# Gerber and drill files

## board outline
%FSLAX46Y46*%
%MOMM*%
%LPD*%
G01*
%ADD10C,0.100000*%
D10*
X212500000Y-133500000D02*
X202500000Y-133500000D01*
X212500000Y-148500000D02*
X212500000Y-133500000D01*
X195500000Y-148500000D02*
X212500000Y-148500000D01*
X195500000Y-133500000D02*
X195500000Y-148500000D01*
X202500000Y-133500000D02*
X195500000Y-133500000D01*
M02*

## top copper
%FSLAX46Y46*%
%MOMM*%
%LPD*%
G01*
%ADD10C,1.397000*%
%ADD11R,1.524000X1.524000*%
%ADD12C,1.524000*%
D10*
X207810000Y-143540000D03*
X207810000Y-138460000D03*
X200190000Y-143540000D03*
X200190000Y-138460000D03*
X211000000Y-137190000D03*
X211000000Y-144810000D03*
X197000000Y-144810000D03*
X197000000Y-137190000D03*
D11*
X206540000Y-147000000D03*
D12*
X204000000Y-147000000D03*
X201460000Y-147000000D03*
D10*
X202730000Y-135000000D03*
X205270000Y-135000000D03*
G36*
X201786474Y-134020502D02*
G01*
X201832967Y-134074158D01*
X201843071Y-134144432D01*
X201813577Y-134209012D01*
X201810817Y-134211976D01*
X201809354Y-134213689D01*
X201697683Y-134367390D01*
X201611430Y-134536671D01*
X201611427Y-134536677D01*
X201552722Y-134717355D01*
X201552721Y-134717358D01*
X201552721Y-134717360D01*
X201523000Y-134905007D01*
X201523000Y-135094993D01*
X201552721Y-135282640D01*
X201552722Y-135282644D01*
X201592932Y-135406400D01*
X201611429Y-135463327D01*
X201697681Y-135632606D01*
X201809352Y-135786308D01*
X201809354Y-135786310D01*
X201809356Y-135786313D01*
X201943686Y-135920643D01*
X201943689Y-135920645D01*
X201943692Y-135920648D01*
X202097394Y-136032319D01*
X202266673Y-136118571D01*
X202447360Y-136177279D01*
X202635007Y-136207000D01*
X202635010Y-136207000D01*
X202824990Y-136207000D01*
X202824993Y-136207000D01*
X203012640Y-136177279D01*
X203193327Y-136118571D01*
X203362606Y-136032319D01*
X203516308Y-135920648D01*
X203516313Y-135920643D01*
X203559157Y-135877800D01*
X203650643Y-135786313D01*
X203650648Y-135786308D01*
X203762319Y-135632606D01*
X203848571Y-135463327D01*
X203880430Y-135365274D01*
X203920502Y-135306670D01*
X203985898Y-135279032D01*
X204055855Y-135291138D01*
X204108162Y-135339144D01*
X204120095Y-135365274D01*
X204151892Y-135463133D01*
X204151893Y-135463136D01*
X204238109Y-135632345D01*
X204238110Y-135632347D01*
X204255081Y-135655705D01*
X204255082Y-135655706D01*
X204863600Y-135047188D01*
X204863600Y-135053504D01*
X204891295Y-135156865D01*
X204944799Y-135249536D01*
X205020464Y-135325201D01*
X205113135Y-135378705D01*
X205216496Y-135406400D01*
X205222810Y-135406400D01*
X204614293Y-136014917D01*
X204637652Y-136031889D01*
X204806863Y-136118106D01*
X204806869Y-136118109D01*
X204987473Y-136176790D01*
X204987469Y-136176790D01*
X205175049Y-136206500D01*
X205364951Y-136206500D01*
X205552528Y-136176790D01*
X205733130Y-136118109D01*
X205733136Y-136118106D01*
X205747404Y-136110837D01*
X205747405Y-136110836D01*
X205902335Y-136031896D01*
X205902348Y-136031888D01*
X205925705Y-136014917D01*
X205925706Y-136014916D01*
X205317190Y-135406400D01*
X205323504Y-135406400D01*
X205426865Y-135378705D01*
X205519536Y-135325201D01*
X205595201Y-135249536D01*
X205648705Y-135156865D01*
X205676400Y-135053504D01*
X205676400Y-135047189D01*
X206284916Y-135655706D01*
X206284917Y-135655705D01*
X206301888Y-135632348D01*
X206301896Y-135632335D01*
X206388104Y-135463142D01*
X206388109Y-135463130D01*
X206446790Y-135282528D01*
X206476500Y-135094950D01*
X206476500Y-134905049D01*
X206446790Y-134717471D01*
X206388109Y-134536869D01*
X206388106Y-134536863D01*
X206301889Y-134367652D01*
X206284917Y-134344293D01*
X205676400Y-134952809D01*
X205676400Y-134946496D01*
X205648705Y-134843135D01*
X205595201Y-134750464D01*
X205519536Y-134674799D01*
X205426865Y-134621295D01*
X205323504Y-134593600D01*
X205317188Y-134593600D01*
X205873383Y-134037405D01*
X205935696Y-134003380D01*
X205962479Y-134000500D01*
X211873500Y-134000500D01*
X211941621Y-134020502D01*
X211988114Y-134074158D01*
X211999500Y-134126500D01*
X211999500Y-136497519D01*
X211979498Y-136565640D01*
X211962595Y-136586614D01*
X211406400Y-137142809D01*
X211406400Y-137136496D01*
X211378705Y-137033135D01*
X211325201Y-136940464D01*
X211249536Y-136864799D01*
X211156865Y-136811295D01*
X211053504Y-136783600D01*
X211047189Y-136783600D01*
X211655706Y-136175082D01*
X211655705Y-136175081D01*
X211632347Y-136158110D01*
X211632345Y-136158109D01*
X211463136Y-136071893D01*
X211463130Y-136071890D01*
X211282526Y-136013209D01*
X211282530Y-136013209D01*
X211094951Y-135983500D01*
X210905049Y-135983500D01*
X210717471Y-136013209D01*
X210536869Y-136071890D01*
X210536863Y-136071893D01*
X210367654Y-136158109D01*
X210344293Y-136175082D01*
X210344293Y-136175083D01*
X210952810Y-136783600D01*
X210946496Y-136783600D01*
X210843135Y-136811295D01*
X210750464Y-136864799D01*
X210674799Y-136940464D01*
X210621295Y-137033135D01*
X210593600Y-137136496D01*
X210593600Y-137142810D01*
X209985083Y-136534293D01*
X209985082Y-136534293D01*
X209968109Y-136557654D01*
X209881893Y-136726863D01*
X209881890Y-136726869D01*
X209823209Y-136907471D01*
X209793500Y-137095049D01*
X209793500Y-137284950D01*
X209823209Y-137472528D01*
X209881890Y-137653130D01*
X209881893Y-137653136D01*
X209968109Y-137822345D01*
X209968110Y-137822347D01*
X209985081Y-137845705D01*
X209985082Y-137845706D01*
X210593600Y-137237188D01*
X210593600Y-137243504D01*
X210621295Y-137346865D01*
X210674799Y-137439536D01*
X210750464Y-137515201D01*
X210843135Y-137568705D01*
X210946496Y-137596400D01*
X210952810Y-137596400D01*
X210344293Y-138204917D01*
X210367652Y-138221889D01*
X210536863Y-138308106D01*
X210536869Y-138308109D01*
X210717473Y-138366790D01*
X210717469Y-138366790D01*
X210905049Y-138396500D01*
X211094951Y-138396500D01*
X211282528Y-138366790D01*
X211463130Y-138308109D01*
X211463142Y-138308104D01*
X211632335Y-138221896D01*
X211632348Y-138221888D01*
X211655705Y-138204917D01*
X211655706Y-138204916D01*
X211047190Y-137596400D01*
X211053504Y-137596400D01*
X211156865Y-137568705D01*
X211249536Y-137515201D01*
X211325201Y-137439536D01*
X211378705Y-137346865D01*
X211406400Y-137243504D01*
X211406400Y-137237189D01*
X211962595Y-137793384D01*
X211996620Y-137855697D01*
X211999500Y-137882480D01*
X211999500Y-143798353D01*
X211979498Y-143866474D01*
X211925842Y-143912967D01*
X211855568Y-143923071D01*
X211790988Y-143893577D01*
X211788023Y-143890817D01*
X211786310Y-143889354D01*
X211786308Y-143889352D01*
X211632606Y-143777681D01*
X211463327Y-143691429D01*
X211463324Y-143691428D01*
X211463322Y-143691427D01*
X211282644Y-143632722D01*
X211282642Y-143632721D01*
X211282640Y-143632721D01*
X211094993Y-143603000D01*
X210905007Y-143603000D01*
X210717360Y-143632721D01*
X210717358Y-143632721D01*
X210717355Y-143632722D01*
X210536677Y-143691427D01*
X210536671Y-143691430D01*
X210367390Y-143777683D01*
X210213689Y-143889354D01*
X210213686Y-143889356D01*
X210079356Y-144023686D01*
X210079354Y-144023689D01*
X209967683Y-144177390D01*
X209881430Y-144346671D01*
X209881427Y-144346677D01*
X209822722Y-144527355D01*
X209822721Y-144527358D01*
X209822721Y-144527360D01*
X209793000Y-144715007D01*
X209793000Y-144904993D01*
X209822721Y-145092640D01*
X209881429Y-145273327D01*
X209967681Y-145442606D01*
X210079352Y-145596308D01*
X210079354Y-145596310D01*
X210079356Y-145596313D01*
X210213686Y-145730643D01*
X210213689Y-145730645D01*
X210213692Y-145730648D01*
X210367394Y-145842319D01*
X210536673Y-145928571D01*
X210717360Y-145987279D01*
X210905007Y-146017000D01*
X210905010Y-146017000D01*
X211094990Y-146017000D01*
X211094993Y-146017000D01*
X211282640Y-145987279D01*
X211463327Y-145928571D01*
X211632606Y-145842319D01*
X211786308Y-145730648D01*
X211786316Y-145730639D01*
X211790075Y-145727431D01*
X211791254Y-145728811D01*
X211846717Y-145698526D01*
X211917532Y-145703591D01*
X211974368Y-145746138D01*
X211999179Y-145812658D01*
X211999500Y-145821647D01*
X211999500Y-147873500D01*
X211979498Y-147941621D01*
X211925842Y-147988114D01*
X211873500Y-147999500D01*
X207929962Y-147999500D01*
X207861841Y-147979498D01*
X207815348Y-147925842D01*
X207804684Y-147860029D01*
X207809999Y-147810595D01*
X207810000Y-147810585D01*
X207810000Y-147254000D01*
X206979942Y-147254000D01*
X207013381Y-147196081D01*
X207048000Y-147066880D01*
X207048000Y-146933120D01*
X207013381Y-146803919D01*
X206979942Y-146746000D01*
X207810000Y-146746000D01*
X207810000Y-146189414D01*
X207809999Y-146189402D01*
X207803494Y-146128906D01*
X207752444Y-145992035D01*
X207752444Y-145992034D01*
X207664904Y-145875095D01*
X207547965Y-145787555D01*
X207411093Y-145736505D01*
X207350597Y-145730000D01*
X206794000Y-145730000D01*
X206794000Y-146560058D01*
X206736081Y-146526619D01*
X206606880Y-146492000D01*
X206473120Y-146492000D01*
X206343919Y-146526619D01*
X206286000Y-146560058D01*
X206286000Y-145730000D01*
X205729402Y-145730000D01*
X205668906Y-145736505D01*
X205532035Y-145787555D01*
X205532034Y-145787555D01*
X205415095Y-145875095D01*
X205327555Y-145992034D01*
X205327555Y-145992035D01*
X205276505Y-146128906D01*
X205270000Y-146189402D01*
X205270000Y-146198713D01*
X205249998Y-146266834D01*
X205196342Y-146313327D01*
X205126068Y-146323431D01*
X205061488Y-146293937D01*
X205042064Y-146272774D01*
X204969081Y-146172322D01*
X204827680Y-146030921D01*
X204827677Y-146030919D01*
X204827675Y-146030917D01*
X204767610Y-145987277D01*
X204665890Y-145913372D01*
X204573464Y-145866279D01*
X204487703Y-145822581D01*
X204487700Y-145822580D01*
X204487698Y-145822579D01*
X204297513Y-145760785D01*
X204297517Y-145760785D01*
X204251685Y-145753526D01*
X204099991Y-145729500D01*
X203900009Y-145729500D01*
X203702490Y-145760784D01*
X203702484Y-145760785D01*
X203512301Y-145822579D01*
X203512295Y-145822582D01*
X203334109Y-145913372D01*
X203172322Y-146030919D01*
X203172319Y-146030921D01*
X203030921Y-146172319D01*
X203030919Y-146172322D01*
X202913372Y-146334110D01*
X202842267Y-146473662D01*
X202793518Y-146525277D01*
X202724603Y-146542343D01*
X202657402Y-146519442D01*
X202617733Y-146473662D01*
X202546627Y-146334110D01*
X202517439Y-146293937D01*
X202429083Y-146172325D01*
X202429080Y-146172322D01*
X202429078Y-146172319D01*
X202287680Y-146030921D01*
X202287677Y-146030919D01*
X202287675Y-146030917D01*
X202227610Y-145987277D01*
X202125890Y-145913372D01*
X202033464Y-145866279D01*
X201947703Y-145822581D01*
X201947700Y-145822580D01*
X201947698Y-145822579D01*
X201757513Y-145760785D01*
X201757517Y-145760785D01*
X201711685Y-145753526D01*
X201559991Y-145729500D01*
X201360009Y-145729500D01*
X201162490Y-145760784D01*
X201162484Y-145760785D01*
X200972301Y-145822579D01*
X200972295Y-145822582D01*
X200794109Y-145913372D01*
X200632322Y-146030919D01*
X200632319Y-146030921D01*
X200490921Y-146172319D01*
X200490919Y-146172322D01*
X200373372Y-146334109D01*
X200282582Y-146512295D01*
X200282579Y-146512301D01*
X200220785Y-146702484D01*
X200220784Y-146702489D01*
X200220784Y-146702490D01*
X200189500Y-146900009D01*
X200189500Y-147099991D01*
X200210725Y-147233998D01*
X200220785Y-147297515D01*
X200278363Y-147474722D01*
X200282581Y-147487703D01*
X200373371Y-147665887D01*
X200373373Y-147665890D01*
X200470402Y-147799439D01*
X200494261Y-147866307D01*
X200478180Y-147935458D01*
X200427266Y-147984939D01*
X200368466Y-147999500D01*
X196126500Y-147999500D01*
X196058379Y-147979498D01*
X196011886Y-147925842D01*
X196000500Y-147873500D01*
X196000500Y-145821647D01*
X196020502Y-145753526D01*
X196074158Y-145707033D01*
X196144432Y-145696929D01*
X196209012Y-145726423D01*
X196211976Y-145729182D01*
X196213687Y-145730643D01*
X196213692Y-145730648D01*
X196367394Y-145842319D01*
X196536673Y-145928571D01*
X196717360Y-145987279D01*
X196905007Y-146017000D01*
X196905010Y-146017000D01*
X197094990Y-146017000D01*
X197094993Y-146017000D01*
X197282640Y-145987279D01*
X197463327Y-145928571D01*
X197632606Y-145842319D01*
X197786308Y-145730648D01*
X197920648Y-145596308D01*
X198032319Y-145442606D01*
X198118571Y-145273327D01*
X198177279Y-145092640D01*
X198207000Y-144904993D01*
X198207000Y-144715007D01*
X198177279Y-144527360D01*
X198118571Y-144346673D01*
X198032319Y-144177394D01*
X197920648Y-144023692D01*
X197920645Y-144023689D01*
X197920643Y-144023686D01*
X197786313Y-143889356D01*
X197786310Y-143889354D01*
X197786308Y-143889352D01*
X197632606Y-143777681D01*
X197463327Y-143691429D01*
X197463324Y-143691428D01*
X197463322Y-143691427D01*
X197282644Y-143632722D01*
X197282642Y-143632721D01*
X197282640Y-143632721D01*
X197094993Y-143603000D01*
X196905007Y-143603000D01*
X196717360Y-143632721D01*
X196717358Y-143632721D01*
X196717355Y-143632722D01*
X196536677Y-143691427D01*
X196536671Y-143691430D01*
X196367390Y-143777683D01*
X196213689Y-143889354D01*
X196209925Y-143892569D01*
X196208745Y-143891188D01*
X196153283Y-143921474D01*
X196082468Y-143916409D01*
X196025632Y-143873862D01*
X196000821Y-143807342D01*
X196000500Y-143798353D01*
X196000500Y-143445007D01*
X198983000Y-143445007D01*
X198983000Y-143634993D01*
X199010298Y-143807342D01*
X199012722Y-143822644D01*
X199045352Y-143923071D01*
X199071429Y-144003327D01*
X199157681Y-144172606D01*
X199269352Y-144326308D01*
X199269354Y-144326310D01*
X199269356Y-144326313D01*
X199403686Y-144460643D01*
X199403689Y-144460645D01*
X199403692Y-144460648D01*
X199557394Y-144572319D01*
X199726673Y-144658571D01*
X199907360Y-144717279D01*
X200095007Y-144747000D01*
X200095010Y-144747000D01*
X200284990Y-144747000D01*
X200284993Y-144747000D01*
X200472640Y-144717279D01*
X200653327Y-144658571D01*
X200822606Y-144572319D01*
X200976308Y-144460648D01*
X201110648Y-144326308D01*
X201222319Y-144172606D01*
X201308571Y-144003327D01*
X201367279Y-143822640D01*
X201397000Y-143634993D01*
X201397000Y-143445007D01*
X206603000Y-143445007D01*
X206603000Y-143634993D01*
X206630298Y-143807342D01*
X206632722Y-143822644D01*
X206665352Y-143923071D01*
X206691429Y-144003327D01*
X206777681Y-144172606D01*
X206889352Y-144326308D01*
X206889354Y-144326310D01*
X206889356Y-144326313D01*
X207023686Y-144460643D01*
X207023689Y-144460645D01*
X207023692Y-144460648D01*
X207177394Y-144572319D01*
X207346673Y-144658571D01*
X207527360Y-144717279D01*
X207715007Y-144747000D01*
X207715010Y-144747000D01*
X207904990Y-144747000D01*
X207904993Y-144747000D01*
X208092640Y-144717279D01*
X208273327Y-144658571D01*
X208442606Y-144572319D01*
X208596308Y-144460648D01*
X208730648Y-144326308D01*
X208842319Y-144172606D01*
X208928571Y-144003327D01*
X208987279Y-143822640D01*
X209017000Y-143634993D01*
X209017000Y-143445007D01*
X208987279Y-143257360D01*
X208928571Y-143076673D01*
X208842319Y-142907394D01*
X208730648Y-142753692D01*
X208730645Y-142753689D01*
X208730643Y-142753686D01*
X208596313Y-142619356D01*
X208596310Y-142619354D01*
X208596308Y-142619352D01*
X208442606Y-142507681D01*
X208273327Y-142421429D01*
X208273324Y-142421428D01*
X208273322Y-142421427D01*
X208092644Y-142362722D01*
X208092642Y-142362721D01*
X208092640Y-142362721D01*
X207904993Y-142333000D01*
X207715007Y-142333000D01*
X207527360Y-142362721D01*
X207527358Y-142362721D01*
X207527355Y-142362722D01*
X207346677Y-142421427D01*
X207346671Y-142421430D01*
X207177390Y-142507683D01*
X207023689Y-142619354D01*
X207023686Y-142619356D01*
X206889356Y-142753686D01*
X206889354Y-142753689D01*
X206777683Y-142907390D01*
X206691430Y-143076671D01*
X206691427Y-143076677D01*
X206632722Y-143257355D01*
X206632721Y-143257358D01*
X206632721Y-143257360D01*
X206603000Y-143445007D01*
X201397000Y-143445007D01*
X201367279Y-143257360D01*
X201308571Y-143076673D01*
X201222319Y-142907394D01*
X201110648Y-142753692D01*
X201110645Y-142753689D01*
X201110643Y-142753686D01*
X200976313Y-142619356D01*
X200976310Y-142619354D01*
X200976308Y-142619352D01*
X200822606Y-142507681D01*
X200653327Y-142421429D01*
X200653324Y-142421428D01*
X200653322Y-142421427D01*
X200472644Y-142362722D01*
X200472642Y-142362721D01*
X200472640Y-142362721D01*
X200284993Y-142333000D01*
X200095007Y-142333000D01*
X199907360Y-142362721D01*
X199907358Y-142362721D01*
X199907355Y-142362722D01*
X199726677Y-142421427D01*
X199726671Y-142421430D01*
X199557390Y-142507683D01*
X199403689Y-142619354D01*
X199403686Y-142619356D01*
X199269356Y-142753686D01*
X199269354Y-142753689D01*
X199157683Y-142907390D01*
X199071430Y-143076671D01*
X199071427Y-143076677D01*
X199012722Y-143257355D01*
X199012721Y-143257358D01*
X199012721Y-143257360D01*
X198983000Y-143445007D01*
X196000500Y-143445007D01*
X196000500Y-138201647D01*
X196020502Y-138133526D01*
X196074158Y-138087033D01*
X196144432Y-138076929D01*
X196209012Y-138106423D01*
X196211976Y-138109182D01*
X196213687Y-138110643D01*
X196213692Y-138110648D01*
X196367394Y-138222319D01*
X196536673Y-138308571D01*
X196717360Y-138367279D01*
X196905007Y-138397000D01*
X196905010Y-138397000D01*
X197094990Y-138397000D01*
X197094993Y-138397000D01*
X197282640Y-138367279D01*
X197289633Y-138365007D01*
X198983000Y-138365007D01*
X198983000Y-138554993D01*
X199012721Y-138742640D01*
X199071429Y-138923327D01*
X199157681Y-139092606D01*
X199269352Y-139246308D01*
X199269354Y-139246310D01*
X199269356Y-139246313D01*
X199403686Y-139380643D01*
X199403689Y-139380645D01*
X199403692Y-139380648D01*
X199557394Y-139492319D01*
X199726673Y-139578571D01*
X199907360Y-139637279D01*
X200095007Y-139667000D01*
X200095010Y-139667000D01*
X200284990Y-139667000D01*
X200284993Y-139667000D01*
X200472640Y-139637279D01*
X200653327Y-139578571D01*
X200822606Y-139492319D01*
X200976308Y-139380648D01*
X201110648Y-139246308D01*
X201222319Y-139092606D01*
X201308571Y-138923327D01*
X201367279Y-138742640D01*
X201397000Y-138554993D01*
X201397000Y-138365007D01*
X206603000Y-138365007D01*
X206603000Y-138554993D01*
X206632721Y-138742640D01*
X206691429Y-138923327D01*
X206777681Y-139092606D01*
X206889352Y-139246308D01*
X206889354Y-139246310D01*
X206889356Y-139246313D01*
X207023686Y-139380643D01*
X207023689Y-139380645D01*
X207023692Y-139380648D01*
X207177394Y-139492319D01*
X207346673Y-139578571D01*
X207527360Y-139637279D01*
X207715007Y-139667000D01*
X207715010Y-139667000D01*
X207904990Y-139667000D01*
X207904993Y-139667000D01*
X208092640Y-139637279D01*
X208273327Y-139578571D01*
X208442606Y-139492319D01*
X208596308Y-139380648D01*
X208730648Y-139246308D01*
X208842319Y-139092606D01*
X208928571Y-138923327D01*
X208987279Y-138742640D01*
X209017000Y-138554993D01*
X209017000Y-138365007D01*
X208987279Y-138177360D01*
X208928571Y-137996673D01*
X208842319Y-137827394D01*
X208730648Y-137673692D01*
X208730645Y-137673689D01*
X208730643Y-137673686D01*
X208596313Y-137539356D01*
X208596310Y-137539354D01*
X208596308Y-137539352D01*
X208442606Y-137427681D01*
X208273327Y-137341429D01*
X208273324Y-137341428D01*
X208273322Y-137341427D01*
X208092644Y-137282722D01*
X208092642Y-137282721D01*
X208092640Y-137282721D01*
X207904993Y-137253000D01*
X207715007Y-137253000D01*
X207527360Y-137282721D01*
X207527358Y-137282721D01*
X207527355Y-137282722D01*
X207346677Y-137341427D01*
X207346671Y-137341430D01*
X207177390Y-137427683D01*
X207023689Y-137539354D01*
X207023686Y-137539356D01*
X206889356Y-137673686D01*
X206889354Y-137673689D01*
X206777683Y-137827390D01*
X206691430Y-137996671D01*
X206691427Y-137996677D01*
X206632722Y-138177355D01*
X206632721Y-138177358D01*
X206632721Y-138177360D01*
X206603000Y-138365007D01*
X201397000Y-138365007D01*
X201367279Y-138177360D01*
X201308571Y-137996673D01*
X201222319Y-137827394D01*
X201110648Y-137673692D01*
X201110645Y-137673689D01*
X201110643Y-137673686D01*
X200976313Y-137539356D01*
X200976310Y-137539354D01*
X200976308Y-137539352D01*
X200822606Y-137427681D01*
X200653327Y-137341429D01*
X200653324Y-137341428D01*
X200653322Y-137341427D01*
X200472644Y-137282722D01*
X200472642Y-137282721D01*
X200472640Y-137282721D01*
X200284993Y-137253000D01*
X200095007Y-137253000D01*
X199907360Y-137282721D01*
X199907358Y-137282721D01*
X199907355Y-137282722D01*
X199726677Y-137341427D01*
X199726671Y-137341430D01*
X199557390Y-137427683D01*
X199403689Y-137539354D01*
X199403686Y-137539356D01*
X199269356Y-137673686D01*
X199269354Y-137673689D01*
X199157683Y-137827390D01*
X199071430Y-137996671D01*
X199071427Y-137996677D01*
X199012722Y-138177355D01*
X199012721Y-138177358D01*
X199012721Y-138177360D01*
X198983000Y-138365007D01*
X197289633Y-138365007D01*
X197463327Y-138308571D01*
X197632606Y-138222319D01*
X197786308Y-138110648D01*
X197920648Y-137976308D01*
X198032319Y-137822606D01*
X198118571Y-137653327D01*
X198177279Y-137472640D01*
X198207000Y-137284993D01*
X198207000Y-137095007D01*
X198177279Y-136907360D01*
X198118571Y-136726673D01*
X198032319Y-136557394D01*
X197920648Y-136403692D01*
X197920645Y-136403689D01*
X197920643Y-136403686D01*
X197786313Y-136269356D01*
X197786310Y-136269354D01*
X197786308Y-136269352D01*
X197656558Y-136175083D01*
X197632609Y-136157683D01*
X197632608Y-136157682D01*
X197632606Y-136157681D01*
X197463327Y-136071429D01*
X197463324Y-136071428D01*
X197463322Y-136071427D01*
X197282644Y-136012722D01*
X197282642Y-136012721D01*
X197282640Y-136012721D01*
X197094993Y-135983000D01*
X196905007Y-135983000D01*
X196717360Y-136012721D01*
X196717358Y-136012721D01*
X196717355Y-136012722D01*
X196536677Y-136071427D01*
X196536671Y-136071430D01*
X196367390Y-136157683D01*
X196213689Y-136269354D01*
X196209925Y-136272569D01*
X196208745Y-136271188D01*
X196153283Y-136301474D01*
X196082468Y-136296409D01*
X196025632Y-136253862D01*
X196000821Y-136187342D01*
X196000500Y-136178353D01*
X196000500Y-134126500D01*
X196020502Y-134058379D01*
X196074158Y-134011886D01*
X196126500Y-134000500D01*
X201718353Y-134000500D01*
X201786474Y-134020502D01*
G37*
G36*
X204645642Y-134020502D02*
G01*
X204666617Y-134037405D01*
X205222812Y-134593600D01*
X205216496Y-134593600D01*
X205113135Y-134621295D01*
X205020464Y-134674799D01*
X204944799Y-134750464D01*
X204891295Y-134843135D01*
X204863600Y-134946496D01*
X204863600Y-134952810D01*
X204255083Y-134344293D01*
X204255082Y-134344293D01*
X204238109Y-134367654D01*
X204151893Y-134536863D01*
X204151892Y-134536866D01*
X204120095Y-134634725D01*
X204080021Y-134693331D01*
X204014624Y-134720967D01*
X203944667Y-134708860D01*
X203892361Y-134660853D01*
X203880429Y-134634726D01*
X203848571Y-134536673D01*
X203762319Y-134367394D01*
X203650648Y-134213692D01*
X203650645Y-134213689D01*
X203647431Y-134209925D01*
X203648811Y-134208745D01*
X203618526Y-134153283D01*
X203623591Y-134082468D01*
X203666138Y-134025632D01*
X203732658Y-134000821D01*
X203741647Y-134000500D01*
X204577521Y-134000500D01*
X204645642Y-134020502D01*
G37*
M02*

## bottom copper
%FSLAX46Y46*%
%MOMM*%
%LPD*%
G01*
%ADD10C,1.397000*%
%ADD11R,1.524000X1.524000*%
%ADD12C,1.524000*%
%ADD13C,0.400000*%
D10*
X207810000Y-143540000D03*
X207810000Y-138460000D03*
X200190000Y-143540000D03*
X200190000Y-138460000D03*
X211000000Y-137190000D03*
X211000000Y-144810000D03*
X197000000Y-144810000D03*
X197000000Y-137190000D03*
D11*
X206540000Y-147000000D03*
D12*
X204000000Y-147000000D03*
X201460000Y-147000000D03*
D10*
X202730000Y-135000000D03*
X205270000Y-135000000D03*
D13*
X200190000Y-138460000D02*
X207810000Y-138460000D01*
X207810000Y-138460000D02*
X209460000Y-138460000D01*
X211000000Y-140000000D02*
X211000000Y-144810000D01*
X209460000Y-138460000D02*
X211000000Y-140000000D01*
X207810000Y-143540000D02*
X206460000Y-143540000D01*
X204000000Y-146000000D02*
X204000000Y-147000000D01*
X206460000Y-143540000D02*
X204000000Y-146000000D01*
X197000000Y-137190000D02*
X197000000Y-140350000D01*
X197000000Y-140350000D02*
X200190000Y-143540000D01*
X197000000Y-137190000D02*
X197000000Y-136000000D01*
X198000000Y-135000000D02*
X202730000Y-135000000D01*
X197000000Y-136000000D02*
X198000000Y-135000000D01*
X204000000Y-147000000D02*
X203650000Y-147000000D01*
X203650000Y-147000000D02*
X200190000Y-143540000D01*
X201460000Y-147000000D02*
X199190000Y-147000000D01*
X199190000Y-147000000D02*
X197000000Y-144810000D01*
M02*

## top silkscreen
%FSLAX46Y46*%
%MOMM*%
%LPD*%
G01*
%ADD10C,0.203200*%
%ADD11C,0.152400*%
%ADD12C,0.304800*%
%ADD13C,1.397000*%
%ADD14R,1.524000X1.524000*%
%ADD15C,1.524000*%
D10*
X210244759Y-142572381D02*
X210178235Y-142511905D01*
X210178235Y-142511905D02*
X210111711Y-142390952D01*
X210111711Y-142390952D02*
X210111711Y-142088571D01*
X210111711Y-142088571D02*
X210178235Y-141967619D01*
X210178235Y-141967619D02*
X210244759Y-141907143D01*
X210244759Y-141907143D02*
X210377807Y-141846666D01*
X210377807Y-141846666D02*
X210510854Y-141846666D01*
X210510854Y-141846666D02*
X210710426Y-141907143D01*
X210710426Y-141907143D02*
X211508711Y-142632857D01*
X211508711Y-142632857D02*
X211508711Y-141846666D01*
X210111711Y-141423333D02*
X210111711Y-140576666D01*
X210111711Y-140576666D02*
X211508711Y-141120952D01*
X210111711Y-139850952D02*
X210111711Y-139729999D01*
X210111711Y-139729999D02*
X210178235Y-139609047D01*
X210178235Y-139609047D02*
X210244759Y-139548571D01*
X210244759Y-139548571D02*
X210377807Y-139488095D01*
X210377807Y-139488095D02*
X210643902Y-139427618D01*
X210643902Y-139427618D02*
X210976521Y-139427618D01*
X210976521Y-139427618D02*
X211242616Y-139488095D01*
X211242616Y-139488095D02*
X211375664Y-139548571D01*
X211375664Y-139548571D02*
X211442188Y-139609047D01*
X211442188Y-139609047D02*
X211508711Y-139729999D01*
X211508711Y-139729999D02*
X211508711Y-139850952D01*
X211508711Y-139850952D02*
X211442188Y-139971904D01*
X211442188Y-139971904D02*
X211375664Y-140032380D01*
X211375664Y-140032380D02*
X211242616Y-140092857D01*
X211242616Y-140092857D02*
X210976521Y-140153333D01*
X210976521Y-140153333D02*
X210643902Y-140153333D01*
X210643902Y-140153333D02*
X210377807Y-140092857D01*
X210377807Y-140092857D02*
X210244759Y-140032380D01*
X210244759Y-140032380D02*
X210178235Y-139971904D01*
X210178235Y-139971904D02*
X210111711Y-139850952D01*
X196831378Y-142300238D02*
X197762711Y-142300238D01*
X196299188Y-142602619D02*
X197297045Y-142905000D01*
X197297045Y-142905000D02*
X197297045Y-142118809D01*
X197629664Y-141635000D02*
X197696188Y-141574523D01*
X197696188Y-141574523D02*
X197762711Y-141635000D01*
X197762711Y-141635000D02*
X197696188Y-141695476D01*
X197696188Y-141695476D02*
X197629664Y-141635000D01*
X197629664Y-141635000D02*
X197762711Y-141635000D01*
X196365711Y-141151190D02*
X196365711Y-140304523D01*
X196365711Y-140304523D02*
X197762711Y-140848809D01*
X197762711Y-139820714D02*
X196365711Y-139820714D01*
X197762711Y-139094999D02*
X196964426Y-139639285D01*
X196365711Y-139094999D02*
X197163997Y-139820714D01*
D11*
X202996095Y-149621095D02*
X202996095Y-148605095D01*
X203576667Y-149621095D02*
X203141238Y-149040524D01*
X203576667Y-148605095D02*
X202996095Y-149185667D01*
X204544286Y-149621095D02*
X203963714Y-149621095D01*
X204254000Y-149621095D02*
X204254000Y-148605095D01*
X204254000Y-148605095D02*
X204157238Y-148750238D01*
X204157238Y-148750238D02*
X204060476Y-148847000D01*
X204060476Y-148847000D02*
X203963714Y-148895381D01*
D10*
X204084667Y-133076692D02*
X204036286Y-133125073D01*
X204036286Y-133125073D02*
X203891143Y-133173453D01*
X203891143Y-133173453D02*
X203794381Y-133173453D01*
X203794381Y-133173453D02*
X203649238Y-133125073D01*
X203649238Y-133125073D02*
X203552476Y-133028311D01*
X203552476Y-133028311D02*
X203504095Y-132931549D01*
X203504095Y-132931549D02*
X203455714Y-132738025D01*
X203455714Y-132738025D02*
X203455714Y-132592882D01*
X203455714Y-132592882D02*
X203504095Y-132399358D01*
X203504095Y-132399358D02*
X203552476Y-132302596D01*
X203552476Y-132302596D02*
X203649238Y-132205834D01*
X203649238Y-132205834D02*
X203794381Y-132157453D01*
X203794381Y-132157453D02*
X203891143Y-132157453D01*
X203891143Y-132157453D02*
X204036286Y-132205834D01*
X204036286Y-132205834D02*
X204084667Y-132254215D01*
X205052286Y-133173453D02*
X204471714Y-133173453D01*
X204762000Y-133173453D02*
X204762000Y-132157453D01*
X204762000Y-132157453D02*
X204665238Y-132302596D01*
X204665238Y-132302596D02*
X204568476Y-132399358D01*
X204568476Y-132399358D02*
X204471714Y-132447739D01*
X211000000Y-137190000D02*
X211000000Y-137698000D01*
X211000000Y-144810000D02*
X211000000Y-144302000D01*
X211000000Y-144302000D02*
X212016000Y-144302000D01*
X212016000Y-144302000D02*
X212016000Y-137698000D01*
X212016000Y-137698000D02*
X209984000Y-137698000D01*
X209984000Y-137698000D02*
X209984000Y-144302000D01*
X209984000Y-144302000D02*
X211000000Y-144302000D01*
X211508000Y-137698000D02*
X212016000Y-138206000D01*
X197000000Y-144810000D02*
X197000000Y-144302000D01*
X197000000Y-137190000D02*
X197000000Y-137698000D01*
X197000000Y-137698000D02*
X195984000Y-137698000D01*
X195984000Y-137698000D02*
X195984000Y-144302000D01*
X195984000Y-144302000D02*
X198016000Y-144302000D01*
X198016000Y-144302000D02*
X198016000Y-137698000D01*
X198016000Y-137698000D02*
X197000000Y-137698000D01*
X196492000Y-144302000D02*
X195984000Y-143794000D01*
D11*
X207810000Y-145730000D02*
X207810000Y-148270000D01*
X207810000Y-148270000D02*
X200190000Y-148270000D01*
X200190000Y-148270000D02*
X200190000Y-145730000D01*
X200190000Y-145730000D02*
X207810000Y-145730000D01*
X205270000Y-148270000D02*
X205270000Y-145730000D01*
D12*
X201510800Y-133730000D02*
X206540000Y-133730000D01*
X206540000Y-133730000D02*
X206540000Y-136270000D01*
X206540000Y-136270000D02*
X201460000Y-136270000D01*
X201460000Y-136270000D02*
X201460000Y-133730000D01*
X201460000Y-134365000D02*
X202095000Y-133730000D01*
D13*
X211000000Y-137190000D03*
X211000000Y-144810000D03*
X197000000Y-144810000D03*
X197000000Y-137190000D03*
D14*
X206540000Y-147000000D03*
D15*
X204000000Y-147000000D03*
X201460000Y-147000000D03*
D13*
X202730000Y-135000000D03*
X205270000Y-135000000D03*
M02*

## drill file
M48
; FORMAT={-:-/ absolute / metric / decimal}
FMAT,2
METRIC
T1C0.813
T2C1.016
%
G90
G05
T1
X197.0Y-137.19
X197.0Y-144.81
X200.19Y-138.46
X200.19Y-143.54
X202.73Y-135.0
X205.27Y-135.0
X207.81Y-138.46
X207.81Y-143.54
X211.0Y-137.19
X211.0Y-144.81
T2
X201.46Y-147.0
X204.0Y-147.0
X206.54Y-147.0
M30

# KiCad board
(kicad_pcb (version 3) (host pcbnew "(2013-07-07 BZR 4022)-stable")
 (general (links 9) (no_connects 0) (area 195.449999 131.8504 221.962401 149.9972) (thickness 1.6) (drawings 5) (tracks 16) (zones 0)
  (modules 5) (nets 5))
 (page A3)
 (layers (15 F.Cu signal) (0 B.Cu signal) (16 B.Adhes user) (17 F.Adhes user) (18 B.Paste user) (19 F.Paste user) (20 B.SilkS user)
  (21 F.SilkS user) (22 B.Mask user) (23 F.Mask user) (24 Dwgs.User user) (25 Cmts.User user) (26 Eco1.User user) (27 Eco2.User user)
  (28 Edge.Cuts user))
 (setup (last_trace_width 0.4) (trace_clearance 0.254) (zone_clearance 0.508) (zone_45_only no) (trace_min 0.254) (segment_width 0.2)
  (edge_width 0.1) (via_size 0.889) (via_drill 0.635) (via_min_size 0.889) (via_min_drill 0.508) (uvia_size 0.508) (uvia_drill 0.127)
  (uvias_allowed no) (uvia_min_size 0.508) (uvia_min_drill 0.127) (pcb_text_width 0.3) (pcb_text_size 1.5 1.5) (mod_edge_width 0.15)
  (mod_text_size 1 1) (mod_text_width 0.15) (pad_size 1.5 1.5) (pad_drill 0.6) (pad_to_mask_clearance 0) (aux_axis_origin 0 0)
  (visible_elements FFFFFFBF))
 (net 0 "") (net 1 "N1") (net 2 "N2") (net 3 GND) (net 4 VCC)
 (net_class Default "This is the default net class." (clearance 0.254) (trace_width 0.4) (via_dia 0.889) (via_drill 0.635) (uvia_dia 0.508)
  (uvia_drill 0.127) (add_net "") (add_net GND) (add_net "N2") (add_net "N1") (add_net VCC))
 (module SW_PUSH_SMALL (layer B.Cu) (at 204 141)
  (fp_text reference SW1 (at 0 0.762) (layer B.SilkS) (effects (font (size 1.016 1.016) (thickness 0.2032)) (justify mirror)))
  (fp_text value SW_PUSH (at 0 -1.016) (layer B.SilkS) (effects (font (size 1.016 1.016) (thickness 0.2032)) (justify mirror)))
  (pad 1 thru_hole circle (at 3.81 2.54) (size 1.397 1.397) (drill 0.8128) (layers *.Cu *.Mask B.SilkS) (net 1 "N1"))
  (pad 2 thru_hole circle (at 3.81 -2.54) (size 1.397 1.397) (drill 0.8128) (layers *.Cu *.Mask B.SilkS) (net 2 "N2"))
  (pad 1 thru_hole circle (at -3.81 2.54) (size 1.397 1.397) (drill 0.8128) (layers *.Cu *.Mask B.SilkS) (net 1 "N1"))
  (pad 2 thru_hole circle (at -3.81 -2.54) (size 1.397 1.397) (drill 0.8128) (layers *.Cu *.Mask B.SilkS) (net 2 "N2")))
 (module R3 (layer F.Cu) (at 211 141 270) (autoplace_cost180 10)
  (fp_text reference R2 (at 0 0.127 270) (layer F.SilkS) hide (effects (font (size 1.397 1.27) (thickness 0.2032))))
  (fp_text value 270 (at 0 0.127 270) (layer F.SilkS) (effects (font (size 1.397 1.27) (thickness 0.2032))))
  (fp_line (start -3.81 0) (end -3.302 0) (layer F.SilkS) (width 0.2032))
  (fp_line (start 3.81 0) (end 3.302 0) (layer F.SilkS) (width 0.2032))
  (fp_line (start 3.302 0) (end 3.302 -1.016) (layer F.SilkS) (width 0.2032))
  (fp_line (start 3.302 -1.016) (end -3.302 -1.016) (layer F.SilkS) (width 0.2032))
  (fp_line (start -3.302 -1.016) (end -3.302 1.016) (layer F.SilkS) (width 0.2032))
  (fp_line (start -3.302 1.016) (end 3.302 1.016) (layer F.SilkS) (width 0.2032))
  (fp_line (start 3.302 1.016) (end 3.302 0) (layer F.SilkS) (width 0.2032))
  (fp_line (start -3.302 -0.508) (end -2.794 -1.016) (layer F.SilkS) (width 0.2032))
  (pad 1 thru_hole circle (at -3.81 0 270) (size 1.397 1.397) (drill 0.8128) (layers *.Cu *.Mask F.SilkS) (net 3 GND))
  (pad 2 thru_hole circle (at 3.81 0 270) (size 1.397 1.397) (drill 0.8128) (layers *.Cu *.Mask F.SilkS) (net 2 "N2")))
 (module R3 (layer F.Cu) (at 197 141 90) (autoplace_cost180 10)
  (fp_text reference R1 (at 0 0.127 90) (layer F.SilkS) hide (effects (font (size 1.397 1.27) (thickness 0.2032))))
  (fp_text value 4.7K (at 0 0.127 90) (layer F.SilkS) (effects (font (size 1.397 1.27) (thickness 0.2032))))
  (fp_line (start -3.81 0) (end -3.302 0) (layer F.SilkS) (width 0.2032))
  (fp_line (start 3.81 0) (end 3.302 0) (layer F.SilkS) (width 0.2032))
  (fp_line (start 3.302 0) (end 3.302 -1.016) (layer F.SilkS) (width 0.2032))
  (fp_line (start 3.302 -1.016) (end -3.302 -1.016) (layer F.SilkS) (width 0.2032))
  (fp_line (start -3.302 -1.016) (end -3.302 1.016) (layer F.SilkS) (width 0.2032))
  (fp_line (start -3.302 1.016) (end 3.302 1.016) (layer F.SilkS) (width 0.2032))
  (fp_line (start 3.302 1.016) (end 3.302 0) (layer F.SilkS) (width 0.2032))
  (fp_line (start -3.302 -0.508) (end -2.794 -1.016) (layer F.SilkS) (width 0.2032))
  (pad 1 thru_hole circle (at -3.81 0 90) (size 1.397 1.397) (drill 0.8128) (layers *.Cu *.Mask F.SilkS) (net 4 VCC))
  (pad 2 thru_hole circle (at 3.81 0 90) (size 1.397 1.397) (drill 0.8128) (layers *.Cu *.Mask F.SilkS) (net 1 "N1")))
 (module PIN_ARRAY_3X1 (layer F.Cu) (at 204 147 180)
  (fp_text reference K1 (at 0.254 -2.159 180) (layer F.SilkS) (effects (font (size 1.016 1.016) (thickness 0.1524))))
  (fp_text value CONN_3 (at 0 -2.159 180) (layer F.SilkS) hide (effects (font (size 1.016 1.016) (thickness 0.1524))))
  (fp_line (start -3.81 1.27) (end -3.81 -1.27) (layer F.SilkS) (width 0.1524))
  (fp_line (start -3.81 -1.27) (end 3.81 -1.27) (layer F.SilkS) (width 0.1524))
  (fp_line (start 3.81 -1.27) (end 3.81 1.27) (layer F.SilkS) (width 0.1524))
  (fp_line (start 3.81 1.27) (end -3.81 1.27) (layer F.SilkS) (width 0.1524))
  (fp_line (start -1.27 -1.27) (end -1.27 1.27) (layer F.SilkS) (width 0.1524))
  (pad 1 thru_hole rect (at -2.54 0 180) (size 1.524 1.524) (drill 1.016) (layers *.Cu *.Mask F.SilkS) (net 3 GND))
  (pad 2 thru_hole circle (at 0 0 180) (size 1.524 1.524) (drill 1.016) (layers *.Cu *.Mask F.SilkS) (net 1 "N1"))
  (pad 3 thru_hole circle (at 2.54 0 180) (size 1.524 1.524) (drill 1.016) (layers *.Cu *.Mask F.SilkS) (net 4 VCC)))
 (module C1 (layer F.Cu) (at 204 135)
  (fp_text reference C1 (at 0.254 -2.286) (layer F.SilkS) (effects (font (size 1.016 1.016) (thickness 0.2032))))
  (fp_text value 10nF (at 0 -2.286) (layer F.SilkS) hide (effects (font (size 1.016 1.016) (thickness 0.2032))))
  (fp_line (start -2.4892 -1.27) (end 2.54 -1.27) (layer F.SilkS) (width 0.3048))
  (fp_line (start 2.54 -1.27) (end 2.54 1.27) (layer F.SilkS) (width 0.3048))
  (fp_line (start 2.54 1.27) (end -2.54 1.27) (layer F.SilkS) (width 0.3048))
  (fp_line (start -2.54 1.27) (end -2.54 -1.27) (layer F.SilkS) (width 0.3048))
  (fp_line (start -2.54 -0.635) (end -1.905 -1.27) (layer F.SilkS) (width 0.3048))
  (pad 1 thru_hole circle (at -1.27 0) (size 1.397 1.397) (drill 0.8128) (layers *.Cu *.Mask F.SilkS) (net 1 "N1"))
  (pad 2 thru_hole circle (at 1.27 0) (size 1.397 1.397) (drill 0.8128) (layers *.Cu *.Mask F.SilkS) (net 3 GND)))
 (gr_line (start 212.5 133.5) (end 202.5 133.5) (angle 90) (layer Edge.Cuts) (width 0.1))
 (gr_line (start 212.5 148.5) (end 212.5 133.5) (angle 90) (layer Edge.Cuts) (width 0.1))
 (gr_line (start 195.5 148.5) (end 212.5 148.5) (angle 90) (layer Edge.Cuts) (width 0.1))
 (gr_line (start 195.5 133.5) (end 195.5 148.5) (angle 90) (layer Edge.Cuts) (width 0.1))
 (gr_line (start 202.5 133.5) (end 195.5 133.5) (angle 90) (layer Edge.Cuts) (width 0.1))
 (segment (start 200.19 138.46) (end 207.81 138.46) (width 0.4) (layer B.Cu) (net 2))
 (segment (start 207.81 138.46) (end 209.46 138.46) (width 0.4) (layer B.Cu) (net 2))
 (segment (start 211 140) (end 211 144.81) (width 0.4) (layer B.Cu) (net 2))
 (segment (start 209.46 138.46) (end 211 140) (width 0.4) (layer B.Cu) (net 2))
 (segment (start 207.81 143.54) (end 206.46 143.54) (width 0.4) (layer B.Cu) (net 1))
 (segment (start 204 146) (end 204 147) (width 0.4) (layer B.Cu) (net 1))
 (segment (start 206.46 143.54) (end 204 146) (width 0.4) (layer B.Cu) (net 1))
 (segment (start 197 137.19) (end 197 140.35) (width 0.4) (layer B.Cu) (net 1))
 (segment (start 197 140.35) (end 200.19 143.54) (width 0.4) (layer B.Cu) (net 1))
 (segment (start 197 137.19) (end 197 136) (width 0.4) (layer B.Cu) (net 1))
 (segment (start 198 135) (end 202.73 135) (width 0.4) (layer B.Cu) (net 1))
 (segment (start 197 136) (end 198 135) (width 0.4) (layer B.Cu) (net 1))
 (segment (start 204 147) (end 203.65 147) (width 0.4) (layer B.Cu) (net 1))
 (segment (start 203.65 147) (end 200.19 143.54) (width 0.4) (layer B.Cu) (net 1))
 (segment (start 201.46 147) (end 199.19 147) (width 0.4) (layer B.Cu) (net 4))
 (segment (start 199.19 147) (end 197 144.81) (width 0.4) (layer B.Cu) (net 4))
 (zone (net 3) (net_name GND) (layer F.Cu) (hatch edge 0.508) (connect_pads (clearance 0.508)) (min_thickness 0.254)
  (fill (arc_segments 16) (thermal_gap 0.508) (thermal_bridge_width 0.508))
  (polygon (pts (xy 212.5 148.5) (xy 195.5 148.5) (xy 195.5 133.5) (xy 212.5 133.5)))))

